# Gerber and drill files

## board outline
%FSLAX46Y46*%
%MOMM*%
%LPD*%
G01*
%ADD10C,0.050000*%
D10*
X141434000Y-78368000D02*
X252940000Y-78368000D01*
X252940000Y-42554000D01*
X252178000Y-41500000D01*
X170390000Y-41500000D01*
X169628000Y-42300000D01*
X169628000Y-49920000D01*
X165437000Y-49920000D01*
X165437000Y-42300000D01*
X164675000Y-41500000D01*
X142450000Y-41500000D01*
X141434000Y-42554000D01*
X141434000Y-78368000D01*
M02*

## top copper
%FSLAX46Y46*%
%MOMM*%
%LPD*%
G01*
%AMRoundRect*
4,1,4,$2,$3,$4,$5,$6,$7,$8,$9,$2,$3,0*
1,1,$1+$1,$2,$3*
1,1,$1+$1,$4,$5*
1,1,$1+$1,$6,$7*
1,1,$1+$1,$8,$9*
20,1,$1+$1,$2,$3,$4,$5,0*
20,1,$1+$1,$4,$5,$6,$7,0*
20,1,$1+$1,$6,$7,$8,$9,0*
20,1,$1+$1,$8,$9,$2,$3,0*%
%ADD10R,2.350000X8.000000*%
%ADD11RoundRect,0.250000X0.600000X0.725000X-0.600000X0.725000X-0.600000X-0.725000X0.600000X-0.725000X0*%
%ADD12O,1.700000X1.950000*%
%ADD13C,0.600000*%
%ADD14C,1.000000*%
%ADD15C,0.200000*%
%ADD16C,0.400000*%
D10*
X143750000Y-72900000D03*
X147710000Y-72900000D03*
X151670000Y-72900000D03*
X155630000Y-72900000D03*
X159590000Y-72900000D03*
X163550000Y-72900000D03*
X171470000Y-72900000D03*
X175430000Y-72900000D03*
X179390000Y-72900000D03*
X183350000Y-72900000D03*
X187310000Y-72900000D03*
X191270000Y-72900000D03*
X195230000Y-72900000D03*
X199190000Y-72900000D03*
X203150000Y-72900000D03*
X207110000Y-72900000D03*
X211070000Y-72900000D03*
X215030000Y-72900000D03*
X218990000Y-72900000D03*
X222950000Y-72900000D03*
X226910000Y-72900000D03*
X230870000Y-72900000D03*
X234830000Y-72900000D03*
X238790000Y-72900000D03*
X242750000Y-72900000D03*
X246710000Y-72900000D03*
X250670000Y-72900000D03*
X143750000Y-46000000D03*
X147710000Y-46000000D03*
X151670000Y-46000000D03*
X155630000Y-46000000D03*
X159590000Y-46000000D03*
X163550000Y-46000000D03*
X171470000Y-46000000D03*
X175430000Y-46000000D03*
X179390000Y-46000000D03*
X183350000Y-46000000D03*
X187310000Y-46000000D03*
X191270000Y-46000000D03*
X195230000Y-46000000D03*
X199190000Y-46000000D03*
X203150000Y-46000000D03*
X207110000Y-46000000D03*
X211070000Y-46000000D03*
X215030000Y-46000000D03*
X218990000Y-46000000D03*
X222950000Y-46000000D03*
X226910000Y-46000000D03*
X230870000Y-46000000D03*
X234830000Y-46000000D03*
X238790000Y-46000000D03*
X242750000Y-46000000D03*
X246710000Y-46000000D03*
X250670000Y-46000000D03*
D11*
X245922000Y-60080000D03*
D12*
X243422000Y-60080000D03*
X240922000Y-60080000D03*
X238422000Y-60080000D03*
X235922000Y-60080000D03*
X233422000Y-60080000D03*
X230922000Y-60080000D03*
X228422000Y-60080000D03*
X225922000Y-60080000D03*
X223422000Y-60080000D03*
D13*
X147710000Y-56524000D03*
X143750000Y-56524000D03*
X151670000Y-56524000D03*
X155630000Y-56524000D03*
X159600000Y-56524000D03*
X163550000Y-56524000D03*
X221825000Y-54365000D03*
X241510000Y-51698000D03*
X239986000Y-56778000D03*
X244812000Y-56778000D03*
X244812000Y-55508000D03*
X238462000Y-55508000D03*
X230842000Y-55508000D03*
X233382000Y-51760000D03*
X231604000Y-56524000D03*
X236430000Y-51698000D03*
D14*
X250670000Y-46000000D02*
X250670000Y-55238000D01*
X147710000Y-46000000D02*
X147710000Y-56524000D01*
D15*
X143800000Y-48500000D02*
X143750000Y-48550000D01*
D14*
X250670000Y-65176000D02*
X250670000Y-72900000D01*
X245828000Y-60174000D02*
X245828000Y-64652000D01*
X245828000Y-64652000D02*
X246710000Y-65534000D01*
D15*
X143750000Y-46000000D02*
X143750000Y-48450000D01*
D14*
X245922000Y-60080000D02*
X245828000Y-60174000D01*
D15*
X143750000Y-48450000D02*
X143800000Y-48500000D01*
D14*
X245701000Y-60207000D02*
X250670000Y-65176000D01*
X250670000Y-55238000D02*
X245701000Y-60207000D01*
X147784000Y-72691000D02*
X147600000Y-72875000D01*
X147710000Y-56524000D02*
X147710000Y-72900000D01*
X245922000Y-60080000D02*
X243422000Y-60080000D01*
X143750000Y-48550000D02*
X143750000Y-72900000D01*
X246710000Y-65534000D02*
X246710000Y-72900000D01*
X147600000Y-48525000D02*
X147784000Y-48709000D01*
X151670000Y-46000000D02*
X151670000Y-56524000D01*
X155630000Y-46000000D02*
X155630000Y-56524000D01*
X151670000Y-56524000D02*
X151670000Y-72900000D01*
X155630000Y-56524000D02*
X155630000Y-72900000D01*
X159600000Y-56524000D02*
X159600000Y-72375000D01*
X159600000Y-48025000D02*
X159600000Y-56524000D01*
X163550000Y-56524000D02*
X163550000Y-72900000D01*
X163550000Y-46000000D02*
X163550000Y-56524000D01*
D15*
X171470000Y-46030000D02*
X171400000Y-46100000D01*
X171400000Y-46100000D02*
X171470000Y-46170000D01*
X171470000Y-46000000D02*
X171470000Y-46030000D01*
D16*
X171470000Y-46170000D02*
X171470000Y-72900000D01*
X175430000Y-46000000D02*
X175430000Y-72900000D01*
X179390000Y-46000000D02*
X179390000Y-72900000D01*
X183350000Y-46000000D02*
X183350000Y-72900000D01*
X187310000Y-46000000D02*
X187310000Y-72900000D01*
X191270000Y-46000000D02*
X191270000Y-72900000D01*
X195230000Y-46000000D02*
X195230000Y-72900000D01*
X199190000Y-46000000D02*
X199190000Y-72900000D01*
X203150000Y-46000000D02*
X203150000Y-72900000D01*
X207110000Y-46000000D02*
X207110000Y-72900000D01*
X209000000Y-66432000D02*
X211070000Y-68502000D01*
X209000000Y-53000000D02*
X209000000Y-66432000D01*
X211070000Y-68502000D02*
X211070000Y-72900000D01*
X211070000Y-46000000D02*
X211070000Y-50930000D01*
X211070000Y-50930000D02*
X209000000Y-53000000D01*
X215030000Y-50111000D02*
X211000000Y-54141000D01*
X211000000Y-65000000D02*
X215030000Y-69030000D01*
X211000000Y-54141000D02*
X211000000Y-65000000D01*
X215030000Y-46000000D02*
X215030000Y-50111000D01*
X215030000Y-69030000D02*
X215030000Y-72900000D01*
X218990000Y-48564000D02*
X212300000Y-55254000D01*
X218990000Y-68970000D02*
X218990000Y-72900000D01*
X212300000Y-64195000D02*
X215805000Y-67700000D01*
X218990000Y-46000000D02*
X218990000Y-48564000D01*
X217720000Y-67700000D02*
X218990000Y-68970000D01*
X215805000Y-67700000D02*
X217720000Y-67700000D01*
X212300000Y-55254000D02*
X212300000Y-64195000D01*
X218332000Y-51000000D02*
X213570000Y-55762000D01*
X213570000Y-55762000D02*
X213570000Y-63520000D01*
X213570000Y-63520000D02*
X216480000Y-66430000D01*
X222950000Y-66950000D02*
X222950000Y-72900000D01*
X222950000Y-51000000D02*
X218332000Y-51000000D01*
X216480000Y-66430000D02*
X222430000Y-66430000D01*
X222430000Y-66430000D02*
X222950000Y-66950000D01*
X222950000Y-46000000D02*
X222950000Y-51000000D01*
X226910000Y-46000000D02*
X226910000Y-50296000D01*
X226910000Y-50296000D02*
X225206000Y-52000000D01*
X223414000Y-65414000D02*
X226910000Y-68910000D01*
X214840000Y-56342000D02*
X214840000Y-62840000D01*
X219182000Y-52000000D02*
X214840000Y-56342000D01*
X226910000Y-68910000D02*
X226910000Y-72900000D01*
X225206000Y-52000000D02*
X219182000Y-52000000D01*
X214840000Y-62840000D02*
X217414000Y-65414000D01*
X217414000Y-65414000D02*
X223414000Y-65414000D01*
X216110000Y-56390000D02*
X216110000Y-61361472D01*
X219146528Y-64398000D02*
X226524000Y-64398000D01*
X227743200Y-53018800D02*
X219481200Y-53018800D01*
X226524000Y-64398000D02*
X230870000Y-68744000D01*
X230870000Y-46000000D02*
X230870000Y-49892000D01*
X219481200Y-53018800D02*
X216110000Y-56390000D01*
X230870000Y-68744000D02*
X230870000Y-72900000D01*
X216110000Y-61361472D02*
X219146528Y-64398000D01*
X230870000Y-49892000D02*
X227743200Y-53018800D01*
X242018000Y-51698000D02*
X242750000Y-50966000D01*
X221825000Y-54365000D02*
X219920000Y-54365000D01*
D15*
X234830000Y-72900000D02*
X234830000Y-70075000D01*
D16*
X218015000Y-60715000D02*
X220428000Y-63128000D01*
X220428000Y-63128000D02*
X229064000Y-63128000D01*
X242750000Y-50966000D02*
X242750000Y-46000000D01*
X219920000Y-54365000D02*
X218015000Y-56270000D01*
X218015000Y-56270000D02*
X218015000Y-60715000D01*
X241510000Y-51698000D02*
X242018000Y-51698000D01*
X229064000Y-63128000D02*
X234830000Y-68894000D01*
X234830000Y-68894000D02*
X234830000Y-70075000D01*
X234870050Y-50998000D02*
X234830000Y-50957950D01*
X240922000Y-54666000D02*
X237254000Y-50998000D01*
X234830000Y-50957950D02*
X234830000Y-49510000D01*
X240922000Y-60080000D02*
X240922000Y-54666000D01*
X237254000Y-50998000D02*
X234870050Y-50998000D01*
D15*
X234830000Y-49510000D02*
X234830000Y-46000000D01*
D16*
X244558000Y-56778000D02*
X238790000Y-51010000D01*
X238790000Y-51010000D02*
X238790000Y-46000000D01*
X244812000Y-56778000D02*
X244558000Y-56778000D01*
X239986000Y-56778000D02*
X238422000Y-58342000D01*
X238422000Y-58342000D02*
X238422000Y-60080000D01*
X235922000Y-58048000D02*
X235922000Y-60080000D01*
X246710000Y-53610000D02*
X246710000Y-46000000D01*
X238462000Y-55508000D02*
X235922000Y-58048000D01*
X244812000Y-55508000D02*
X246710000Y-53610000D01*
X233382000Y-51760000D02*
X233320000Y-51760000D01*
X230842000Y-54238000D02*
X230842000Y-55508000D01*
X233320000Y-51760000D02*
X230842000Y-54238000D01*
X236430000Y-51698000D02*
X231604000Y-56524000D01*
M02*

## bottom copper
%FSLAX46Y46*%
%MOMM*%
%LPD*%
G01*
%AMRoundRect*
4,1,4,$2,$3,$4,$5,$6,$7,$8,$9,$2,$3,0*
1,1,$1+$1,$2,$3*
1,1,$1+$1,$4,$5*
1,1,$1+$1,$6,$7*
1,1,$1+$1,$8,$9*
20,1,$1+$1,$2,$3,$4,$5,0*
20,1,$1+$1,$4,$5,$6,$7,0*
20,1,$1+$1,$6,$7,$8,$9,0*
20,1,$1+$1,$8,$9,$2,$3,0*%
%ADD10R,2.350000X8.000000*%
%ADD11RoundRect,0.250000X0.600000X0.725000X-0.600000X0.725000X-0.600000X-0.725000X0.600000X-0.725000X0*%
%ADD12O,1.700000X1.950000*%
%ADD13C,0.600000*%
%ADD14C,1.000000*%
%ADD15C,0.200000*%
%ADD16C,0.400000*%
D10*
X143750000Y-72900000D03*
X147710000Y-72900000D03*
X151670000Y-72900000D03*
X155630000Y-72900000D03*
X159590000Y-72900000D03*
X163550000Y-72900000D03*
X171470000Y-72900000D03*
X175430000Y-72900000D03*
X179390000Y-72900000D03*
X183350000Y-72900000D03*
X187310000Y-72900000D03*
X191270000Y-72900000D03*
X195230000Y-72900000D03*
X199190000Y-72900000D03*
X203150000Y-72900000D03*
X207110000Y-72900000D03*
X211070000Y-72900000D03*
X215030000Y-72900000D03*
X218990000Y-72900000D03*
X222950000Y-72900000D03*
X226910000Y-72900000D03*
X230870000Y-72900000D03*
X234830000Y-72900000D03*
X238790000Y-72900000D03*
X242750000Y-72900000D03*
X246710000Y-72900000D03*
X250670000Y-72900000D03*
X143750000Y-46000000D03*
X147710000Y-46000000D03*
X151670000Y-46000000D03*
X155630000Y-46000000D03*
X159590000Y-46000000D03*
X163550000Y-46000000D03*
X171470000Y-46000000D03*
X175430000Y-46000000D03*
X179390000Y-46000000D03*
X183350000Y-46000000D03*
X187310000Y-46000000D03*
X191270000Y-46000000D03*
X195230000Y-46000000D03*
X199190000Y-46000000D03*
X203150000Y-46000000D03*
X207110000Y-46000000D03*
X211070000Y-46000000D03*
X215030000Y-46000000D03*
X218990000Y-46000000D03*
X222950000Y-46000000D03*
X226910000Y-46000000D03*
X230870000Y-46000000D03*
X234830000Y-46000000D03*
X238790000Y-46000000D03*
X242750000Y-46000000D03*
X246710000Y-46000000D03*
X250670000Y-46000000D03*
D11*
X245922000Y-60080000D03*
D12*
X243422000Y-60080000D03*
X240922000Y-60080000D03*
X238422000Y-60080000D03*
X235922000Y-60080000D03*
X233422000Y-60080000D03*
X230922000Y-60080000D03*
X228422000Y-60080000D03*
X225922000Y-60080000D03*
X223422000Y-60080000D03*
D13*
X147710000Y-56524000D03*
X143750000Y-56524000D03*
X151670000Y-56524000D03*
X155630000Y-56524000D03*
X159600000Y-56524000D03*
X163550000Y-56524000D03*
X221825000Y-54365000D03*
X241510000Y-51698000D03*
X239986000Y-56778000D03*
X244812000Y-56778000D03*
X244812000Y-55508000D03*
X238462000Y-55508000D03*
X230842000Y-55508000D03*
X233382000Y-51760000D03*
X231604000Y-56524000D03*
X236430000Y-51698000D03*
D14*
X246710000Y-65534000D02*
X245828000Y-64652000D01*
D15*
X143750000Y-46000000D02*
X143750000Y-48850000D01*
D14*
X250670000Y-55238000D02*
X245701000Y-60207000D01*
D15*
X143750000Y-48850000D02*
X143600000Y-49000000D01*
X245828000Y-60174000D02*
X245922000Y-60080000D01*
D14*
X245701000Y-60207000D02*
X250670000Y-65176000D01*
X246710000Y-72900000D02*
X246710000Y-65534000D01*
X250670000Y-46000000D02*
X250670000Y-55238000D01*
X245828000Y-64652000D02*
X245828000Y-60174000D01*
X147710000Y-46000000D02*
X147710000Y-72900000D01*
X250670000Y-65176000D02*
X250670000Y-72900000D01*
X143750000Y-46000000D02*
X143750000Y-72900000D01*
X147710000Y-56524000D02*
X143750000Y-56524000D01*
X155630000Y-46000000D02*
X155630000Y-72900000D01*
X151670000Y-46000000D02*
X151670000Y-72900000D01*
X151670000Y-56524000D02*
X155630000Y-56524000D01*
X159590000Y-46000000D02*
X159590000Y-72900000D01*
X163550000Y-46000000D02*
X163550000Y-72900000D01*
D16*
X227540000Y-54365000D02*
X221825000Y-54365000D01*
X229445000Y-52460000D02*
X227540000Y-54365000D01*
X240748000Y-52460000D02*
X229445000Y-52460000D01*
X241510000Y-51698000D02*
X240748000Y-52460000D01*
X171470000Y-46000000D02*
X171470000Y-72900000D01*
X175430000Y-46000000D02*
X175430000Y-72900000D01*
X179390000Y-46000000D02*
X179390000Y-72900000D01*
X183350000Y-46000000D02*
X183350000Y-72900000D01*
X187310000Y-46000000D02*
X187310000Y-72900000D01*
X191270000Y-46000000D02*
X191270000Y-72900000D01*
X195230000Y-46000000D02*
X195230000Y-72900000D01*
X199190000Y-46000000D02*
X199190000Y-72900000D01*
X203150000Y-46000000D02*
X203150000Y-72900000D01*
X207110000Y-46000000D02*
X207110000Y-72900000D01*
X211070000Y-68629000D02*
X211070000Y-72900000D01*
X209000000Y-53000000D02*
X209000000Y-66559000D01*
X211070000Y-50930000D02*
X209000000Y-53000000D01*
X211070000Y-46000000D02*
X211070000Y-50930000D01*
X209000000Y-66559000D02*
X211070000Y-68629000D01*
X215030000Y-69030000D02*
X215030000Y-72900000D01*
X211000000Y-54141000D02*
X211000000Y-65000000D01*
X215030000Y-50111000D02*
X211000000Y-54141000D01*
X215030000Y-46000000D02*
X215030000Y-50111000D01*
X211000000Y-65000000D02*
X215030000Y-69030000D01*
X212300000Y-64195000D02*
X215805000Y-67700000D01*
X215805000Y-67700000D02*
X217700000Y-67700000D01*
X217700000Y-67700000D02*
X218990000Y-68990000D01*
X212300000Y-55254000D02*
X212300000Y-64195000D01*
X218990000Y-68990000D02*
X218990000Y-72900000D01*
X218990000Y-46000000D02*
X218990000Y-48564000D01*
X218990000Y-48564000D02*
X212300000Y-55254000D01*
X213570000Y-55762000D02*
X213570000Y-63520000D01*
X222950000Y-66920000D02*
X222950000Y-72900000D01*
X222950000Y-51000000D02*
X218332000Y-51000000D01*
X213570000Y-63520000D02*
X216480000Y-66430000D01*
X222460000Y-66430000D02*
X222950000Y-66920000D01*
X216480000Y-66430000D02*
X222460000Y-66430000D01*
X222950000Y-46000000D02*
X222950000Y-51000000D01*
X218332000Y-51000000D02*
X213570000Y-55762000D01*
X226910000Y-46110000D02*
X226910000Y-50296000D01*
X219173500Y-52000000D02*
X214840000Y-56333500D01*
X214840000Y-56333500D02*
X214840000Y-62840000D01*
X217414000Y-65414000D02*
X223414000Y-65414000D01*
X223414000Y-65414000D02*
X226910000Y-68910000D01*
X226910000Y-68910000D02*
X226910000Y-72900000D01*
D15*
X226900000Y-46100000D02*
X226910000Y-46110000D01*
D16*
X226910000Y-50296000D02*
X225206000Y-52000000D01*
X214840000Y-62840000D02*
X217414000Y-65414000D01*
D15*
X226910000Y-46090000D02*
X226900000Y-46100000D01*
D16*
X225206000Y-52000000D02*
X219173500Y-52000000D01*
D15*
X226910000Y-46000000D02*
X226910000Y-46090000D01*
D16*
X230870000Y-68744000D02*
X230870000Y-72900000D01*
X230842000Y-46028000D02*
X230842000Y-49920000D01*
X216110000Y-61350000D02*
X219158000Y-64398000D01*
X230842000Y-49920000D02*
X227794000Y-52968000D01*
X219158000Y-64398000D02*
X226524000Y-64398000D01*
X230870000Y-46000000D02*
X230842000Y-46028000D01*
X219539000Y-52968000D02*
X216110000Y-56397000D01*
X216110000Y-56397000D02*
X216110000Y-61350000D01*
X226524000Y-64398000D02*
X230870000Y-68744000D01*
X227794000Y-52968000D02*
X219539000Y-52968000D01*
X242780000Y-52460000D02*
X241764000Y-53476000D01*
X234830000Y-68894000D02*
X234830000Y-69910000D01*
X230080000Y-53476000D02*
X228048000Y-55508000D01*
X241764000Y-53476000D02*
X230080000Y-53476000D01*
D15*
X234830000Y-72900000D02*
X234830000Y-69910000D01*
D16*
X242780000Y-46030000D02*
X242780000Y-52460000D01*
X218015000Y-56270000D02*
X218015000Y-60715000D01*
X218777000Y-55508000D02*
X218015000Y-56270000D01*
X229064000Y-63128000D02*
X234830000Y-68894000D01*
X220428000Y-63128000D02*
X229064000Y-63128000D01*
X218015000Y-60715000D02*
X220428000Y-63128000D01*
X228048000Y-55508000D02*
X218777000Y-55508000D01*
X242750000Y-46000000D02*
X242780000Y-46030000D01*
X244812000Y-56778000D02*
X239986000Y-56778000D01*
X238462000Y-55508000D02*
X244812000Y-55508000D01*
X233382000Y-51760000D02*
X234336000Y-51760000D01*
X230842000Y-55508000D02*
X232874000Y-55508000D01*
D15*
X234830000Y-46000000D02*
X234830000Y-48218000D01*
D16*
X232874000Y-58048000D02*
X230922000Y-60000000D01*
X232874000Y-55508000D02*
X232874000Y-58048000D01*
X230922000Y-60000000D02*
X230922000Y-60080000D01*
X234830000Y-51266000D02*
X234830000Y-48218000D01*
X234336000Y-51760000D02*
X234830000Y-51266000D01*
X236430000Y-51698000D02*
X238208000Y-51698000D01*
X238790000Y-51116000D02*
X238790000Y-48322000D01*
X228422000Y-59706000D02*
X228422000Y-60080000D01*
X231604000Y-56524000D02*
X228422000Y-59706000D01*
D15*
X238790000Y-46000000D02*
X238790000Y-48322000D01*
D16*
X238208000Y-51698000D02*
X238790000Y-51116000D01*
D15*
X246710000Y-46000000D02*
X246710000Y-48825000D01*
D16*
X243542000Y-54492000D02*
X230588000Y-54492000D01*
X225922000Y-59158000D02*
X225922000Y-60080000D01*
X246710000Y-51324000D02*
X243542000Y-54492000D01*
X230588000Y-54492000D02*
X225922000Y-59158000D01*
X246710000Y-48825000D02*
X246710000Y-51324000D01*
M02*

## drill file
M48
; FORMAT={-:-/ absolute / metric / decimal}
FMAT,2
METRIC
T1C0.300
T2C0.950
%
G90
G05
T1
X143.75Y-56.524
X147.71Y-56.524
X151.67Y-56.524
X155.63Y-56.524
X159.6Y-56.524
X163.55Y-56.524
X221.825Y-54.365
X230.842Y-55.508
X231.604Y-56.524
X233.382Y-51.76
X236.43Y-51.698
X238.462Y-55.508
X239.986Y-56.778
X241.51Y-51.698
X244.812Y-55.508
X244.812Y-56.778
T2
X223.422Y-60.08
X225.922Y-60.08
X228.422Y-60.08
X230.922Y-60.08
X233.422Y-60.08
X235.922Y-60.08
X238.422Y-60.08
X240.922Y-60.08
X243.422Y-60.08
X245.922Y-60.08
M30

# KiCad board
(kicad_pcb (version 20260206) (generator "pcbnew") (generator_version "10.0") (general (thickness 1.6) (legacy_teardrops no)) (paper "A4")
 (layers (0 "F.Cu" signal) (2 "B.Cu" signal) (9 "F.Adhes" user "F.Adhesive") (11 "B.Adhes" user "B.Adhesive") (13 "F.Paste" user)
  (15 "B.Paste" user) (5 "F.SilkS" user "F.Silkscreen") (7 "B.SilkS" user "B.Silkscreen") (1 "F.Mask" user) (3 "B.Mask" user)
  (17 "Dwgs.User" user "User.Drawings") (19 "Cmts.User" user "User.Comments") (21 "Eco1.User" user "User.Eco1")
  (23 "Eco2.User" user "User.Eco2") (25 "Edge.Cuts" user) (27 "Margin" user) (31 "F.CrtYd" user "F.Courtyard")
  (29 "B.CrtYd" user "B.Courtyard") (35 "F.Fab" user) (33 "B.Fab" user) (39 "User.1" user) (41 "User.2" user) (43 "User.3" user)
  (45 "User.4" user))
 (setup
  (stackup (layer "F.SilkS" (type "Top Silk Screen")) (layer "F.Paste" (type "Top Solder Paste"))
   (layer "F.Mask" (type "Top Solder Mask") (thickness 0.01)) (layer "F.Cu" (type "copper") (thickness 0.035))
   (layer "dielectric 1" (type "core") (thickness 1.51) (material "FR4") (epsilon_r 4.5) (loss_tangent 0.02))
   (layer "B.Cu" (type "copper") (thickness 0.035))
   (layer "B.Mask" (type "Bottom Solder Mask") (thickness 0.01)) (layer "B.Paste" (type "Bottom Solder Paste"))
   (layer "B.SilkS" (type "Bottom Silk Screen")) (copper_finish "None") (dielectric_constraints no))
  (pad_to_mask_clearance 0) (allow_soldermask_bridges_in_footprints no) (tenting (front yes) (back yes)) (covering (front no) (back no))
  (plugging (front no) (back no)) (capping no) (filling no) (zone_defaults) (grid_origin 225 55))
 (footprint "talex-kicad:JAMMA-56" (layer "F.Cu") (at 198.21 91.9)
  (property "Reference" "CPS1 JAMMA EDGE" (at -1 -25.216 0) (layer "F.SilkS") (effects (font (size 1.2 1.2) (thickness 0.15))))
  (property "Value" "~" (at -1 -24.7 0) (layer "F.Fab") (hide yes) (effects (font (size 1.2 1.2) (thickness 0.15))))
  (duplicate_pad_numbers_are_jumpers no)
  (pad "1" smd rect (at -54.46 -19) (size 2.35 8) (layers "F.Cu" "F.Mask" "F.Paste") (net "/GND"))
  (pad "2" smd rect (at -50.5 -19) (size 2.35 8) (layers "F.Cu" "F.Mask" "F.Paste") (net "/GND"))
  (pad "3" smd rect (at -46.54 -19) (size 2.35 8) (layers "F.Cu" "F.Mask" "F.Paste") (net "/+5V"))
  (pad "4" smd rect (at -42.58 -19) (size 2.35 8) (layers "F.Cu" "F.Mask" "F.Paste") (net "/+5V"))
  (pad "5" smd rect (at -38.62 -19) (size 2.35 8) (layers "F.Cu" "F.Mask" "F.Paste") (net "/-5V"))
  (pad "6" smd rect (at -34.66 -19) (size 2.35 8) (layers "F.Cu" "F.Mask" "F.Paste") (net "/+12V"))
  (pad "8" smd rect (at -26.74 -19) (size 2.35 8) (layers "F.Cu" "F.Mask" "F.Paste") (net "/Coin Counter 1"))
  (pad "9" smd rect (at -22.78 -19) (size 2.35 8) (layers "F.Cu" "F.Mask" "F.Paste") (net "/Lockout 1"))
  (pad "10" smd rect (at -18.82 -19) (size 2.35 8) (layers "F.Cu" "F.Mask" "F.Paste") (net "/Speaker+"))
  (pad "11" smd rect (at -14.86 -19) (size 2.35 8) (layers "F.Cu" "F.Mask" "F.Paste") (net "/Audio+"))
  (pad "12" smd rect (at -10.9 -19) (size 2.35 8) (layers "F.Cu" "F.Mask" "F.Paste") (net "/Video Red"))
  (pad "13" smd rect (at -6.94 -19) (size 2.35 8) (layers "F.Cu" "F.Mask" "F.Paste") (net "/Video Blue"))
  (pad "14" smd rect (at -2.98 -19) (size 2.35 8) (layers "F.Cu" "F.Mask" "F.Paste") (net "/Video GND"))
  (pad "15" smd rect (at 0.98 -19) (size 2.35 8) (layers "F.Cu" "F.Mask" "F.Paste") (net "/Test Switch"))
  (pad "16" smd rect (at 4.94 -19) (size 2.35 8) (layers "F.Cu" "F.Mask" "F.Paste") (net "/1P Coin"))
  (pad "17" smd rect (at 8.9 -19) (size 2.35 8) (layers "F.Cu" "F.Mask" "F.Paste") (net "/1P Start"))
  (pad "18" smd rect (at 12.86 -19) (size 2.35 8) (layers "F.Cu" "F.Mask" "F.Paste") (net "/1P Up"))
  (pad "19" smd rect (at 16.82 -19) (size 2.35 8) (layers "F.Cu" "F.Mask" "F.Paste") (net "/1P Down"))
  (pad "20" smd rect (at 20.78 -19) (size 2.35 8) (layers "F.Cu" "F.Mask" "F.Paste") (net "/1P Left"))
  (pad "21" smd rect (at 24.74 -19) (size 2.35 8) (layers "F.Cu" "F.Mask" "F.Paste") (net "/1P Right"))
  (pad "22" smd rect (at 28.7 -19) (size 2.35 8) (layers "F.Cu" "F.Mask" "F.Paste") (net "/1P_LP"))
  (pad "23" smd rect (at 32.66 -19) (size 2.35 8) (layers "F.Cu" "F.Mask" "F.Paste") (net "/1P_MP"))
  (pad "24" smd rect (at 36.62 -19) (size 2.35 8) (layers "F.Cu" "F.Mask" "F.Paste") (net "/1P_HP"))
  (pad "25" smd rect (at 40.58 -19) (size 2.35 8) (layers "F.Cu" "F.Mask" "F.Paste") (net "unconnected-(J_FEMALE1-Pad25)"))
  (pad "26" smd rect (at 44.54 -19) (size 2.35 8) (layers "F.Cu" "F.Mask" "F.Paste") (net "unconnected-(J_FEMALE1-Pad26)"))
  (pad "27" smd rect (at 48.5 -19) (size 2.35 8) (layers "F.Cu" "F.Mask" "F.Paste") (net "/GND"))
  (pad "28" smd rect (at 52.46 -19) (size 2.35 8) (layers "F.Cu" "F.Mask" "F.Paste") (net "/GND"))
  (pad "A" smd rect (at -54.46 -19) (size 2.35 8) (layers "B.Cu" "B.Mask" "B.Paste") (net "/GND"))
  (pad "B" smd rect (at -50.5 -19) (size 2.35 8) (layers "B.Cu" "B.Mask" "B.Paste") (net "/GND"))
  (pad "C" smd rect (at -46.54 -19) (size 2.35 8) (layers "B.Cu" "B.Mask" "B.Paste") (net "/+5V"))
  (pad "D" smd rect (at -42.58 -19) (size 2.35 8) (layers "B.Cu" "B.Mask" "B.Paste") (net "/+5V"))
  (pad "E" smd rect (at -38.62 -19) (size 2.35 8) (layers "B.Cu" "B.Mask" "B.Paste") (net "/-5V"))
  (pad "F" smd rect (at -34.66 -19) (size 2.35 8) (layers "B.Cu" "B.Mask" "B.Paste") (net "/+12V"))
  (pad "J" smd rect (at -26.74 -19) (size 2.35 8) (layers "B.Cu" "B.Mask" "B.Paste") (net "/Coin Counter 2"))
  (pad "K" smd rect (at -22.78 -19) (size 2.35 8) (layers "B.Cu" "B.Mask" "B.Paste") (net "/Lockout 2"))
  (pad "L" smd rect (at -18.82 -19) (size 2.35 8) (layers "B.Cu" "B.Mask" "B.Paste") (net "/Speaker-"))
  (pad "M" smd rect (at -14.86 -19) (size 2.35 8) (layers "B.Cu" "B.Mask" "B.Paste") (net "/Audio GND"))
  (pad "N" smd rect (at -10.9 -19) (size 2.35 8) (layers "B.Cu" "B.Mask" "B.Paste") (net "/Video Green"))
  (pad "P" smd rect (at -6.94 -19) (size 2.35 8) (layers "B.Cu" "B.Mask" "B.Paste") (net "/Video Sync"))
  (pad "R" smd rect (at -2.98 -19) (size 2.35 8) (layers "B.Cu" "B.Mask" "B.Paste") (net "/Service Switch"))
  (pad "S" smd rect (at 0.98 -19) (size 2.35 8) (layers "B.Cu" "B.Mask" "B.Paste") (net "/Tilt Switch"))
  (pad "T" smd rect (at 4.94 -19) (size 2.35 8) (layers "B.Cu" "B.Mask" "B.Paste") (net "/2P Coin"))
  (pad "U" smd rect (at 8.9 -19) (size 2.35 8) (layers "B.Cu" "B.Mask" "B.Paste") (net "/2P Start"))
  (pad "V" smd rect (at 12.86 -19) (size 2.35 8) (layers "B.Cu" "B.Mask" "B.Paste") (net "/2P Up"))
  (pad "W" smd rect (at 16.82 -19) (size 2.35 8) (layers "B.Cu" "B.Mask" "B.Paste") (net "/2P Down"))
  (pad "X" smd rect (at 20.78 -19) (size 2.35 8) (layers "B.Cu" "B.Mask" "B.Paste") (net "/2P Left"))
  (pad "Y" smd rect (at 24.74 -19) (size 2.35 8) (layers "B.Cu" "B.Mask" "B.Paste") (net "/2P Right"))
  (pad "Z" smd rect (at 28.7 -19) (size 2.35 8) (layers "B.Cu" "B.Mask" "B.Paste") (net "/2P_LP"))
  (pad "a" smd rect (at 32.66 -19) (size 2.35 8) (layers "B.Cu" "B.Mask" "B.Paste") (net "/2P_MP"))
  (pad "b" smd rect (at 36.62 -19) (size 2.35 8) (layers "B.Cu" "B.Mask" "B.Paste") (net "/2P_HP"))
  (pad "c" smd rect (at 40.58 -19) (size 2.35 8) (layers "B.Cu" "B.Mask" "B.Paste") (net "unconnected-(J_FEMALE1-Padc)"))
  (pad "d" smd rect (at 44.54 -19) (size 2.35 8) (layers "B.Cu" "B.Mask" "B.Paste") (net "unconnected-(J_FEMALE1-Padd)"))
  (pad "e" smd rect (at 48.5 -19) (size 2.35 8) (layers "B.Cu" "B.Mask" "B.Paste") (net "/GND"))
  (pad "f" smd rect (at 52.46 -19) (size 2.35 8) (layers "B.Cu" "B.Mask" "B.Paste") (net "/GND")))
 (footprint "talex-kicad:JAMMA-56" (layer "F.Cu") (at 198.21 65)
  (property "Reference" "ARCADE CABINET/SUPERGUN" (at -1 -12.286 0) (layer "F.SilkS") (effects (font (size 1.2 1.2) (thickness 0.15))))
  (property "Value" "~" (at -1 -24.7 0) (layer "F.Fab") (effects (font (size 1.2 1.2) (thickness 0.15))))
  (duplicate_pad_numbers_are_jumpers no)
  (pad "1" smd rect (at -54.46 -19) (size 2.35 8) (layers "F.Cu" "F.Mask" "F.Paste") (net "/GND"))
  (pad "2" smd rect (at -50.5 -19) (size 2.35 8) (layers "F.Cu" "F.Mask" "F.Paste") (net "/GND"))
  (pad "3" smd rect (at -46.54 -19) (size 2.35 8) (layers "F.Cu" "F.Mask" "F.Paste") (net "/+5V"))
  (pad "4" smd rect (at -42.58 -19) (size 2.35 8) (layers "F.Cu" "F.Mask" "F.Paste") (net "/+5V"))
  (pad "5" smd rect (at -38.62 -19) (size 2.35 8) (layers "F.Cu" "F.Mask" "F.Paste") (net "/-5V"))
  (pad "6" smd rect (at -34.66 -19) (size 2.35 8) (layers "F.Cu" "F.Mask" "F.Paste") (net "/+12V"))
  (pad "8" smd rect (at -26.74 -19) (size 2.35 8) (layers "F.Cu" "F.Mask" "F.Paste") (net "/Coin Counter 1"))
  (pad "9" smd rect (at -22.78 -19) (size 2.35 8) (layers "F.Cu" "F.Mask" "F.Paste") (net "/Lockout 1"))
  (pad "10" smd rect (at -18.82 -19) (size 2.35 8) (layers "F.Cu" "F.Mask" "F.Paste") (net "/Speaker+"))
  (pad "11" smd rect (at -14.86 -19) (size 2.35 8) (layers "F.Cu" "F.Mask" "F.Paste") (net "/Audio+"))
  (pad "12" smd rect (at -10.9 -19) (size 2.35 8) (layers "F.Cu" "F.Mask" "F.Paste") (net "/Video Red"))
  (pad "13" smd rect (at -6.94 -19) (size 2.35 8) (layers "F.Cu" "F.Mask" "F.Paste") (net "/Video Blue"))
  (pad "14" smd rect (at -2.98 -19) (size 2.35 8) (layers "F.Cu" "F.Mask" "F.Paste") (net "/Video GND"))
  (pad "15" smd rect (at 0.98 -19) (size 2.35 8) (layers "F.Cu" "F.Mask" "F.Paste") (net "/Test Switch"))
  (pad "16" smd rect (at 4.94 -19) (size 2.35 8) (layers "F.Cu" "F.Mask" "F.Paste") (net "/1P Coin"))
  (pad "17" smd rect (at 8.9 -19) (size 2.35 8) (layers "F.Cu" "F.Mask" "F.Paste") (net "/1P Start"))
  (pad "18" smd rect (at 12.86 -19) (size 2.35 8) (layers "F.Cu" "F.Mask" "F.Paste") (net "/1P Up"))
  (pad "19" smd rect (at 16.82 -19) (size 2.35 8) (layers "F.Cu" "F.Mask" "F.Paste") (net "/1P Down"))
  (pad "20" smd rect (at 20.78 -19) (size 2.35 8) (layers "F.Cu" "F.Mask" "F.Paste") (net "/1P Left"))
  (pad "21" smd rect (at 24.74 -19) (size 2.35 8) (layers "F.Cu" "F.Mask" "F.Paste") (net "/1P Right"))
  (pad "22" smd rect (at 28.7 -19) (size 2.35 8) (layers "F.Cu" "F.Mask" "F.Paste") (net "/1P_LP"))
  (pad "23" smd rect (at 32.66 -19) (size 2.35 8) (layers "F.Cu" "F.Mask" "F.Paste") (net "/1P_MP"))
  (pad "24" smd rect (at 36.62 -19) (size 2.35 8) (layers "F.Cu" "F.Mask" "F.Paste") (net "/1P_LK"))
  (pad "25" smd rect (at 40.58 -19) (size 2.35 8) (layers "F.Cu" "F.Mask" "F.Paste") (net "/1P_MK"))
  (pad "26" smd rect (at 44.54 -19) (size 2.35 8) (layers "F.Cu" "F.Mask" "F.Paste") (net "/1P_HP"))
  (pad "27" smd rect (at 48.5 -19) (size 2.35 8) (layers "F.Cu" "F.Mask" "F.Paste") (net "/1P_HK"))
  (pad "28" smd rect (at 52.46 -19) (size 2.35 8) (layers "F.Cu" "F.Mask" "F.Paste") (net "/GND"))
  (pad "A" smd rect (at -54.46 -19) (size 2.35 8) (layers "B.Cu" "B.Mask" "B.Paste") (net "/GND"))
  (pad "B" smd rect (at -50.5 -19) (size 2.35 8) (layers "B.Cu" "B.Mask" "B.Paste") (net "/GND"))
  (pad "C" smd rect (at -46.54 -19) (size 2.35 8) (layers "B.Cu" "B.Mask" "B.Paste") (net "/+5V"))
  (pad "D" smd rect (at -42.58 -19) (size 2.35 8) (layers "B.Cu" "B.Mask" "B.Paste") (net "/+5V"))
  (pad "E" smd rect (at -38.62 -19) (size 2.35 8) (layers "B.Cu" "B.Mask" "B.Paste") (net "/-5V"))
  (pad "F" smd rect (at -34.66 -19) (size 2.35 8) (layers "B.Cu" "B.Mask" "B.Paste") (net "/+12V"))
  (pad "J" smd rect (at -26.74 -19) (size 2.35 8) (layers "B.Cu" "B.Mask" "B.Paste") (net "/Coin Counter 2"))
  (pad "K" smd rect (at -22.78 -19) (size 2.35 8) (layers "B.Cu" "B.Mask" "B.Paste") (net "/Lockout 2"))
  (pad "L" smd rect (at -18.82 -19) (size 2.35 8) (layers "B.Cu" "B.Mask" "B.Paste") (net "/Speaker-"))
  (pad "M" smd rect (at -14.86 -19) (size 2.35 8) (layers "B.Cu" "B.Mask" "B.Paste") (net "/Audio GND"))
  (pad "N" smd rect (at -10.9 -19) (size 2.35 8) (layers "B.Cu" "B.Mask" "B.Paste") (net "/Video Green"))
  (pad "P" smd rect (at -6.94 -19) (size 2.35 8) (layers "B.Cu" "B.Mask" "B.Paste") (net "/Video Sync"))
  (pad "R" smd rect (at -2.98 -19) (size 2.35 8) (layers "B.Cu" "B.Mask" "B.Paste") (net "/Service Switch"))
  (pad "S" smd rect (at 0.98 -19) (size 2.35 8) (layers "B.Cu" "B.Mask" "B.Paste") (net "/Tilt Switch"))
  (pad "T" smd rect (at 4.94 -19) (size 2.35 8) (layers "B.Cu" "B.Mask" "B.Paste") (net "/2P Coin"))
  (pad "U" smd rect (at 8.9 -19) (size 2.35 8) (layers "B.Cu" "B.Mask" "B.Paste") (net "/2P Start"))
  (pad "V" smd rect (at 12.86 -19) (size 2.35 8) (layers "B.Cu" "B.Mask" "B.Paste") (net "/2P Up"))
  (pad "W" smd rect (at 16.82 -19) (size 2.35 8) (layers "B.Cu" "B.Mask" "B.Paste") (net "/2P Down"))
  (pad "X" smd rect (at 20.78 -19) (size 2.35 8) (layers "B.Cu" "B.Mask" "B.Paste") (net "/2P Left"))
  (pad "Y" smd rect (at 24.74 -19) (size 2.35 8) (layers "B.Cu" "B.Mask" "B.Paste") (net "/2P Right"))
  (pad "Z" smd rect (at 28.7 -19) (size 2.35 8) (layers "B.Cu" "B.Mask" "B.Paste") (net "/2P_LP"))
  (pad "a" smd rect (at 32.66 -19) (size 2.35 8) (layers "B.Cu" "B.Mask" "B.Paste") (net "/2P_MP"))
  (pad "b" smd rect (at 36.62 -19) (size 2.35 8) (layers "B.Cu" "B.Mask" "B.Paste") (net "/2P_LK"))
  (pad "c" smd rect (at 40.58 -19) (size 2.35 8) (layers "B.Cu" "B.Mask" "B.Paste") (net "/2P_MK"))
  (pad "d" smd rect (at 44.54 -19) (size 2.35 8) (layers "B.Cu" "B.Mask" "B.Paste") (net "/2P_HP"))
  (pad "e" smd rect (at 48.5 -19) (size 2.35 8) (layers "B.Cu" "B.Mask" "B.Paste") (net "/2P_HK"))
  (pad "f" smd rect (at 52.46 -19) (size 2.35 8) (layers "B.Cu" "B.Mask" "B.Paste") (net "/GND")))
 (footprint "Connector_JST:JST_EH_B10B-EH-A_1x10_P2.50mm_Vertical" (layer "F.Cu") (at 245.922 60.08 180)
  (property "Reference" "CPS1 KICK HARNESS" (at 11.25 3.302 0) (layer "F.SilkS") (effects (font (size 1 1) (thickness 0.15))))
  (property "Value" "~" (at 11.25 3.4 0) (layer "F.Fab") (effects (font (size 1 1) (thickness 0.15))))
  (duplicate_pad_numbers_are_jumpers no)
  (pad "1" thru_hole roundrect (at 0 0 180) (size 1.7 1.95) (drill 0.95) (layers "*.Cu" "*.Mask") (remove_unused_layers no)
   (roundrect_rratio 0.147059) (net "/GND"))
  (pad "2" thru_hole oval (at 2.5 0 180) (size 1.7 1.95) (drill 0.95) (layers "*.Cu" "*.Mask") (remove_unused_layers no) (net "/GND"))
  (pad "3" thru_hole oval (at 5 0 180) (size 1.7 1.95) (drill 0.95) (layers "*.Cu" "*.Mask") (remove_unused_layers no) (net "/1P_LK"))
  (pad "4" thru_hole oval (at 7.5 0 180) (size 1.7 1.95) (drill 0.95) (layers "*.Cu" "*.Mask") (remove_unused_layers no) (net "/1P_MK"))
  (pad "5" thru_hole oval (at 10 0 180) (size 1.7 1.95) (drill 0.95) (layers "*.Cu" "*.Mask") (remove_unused_layers no) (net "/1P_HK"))
  (pad "6" thru_hole oval (at 12.5 0 180) (size 1.7 1.95) (drill 0.95) (layers "*.Cu" "*.Mask") (remove_unused_layers no)
   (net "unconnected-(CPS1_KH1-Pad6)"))
  (pad "7" thru_hole oval (at 15 0 180) (size 1.7 1.95) (drill 0.95) (layers "*.Cu" "*.Mask") (remove_unused_layers no) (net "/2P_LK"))
  (pad "8" thru_hole oval (at 17.5 0 180) (size 1.7 1.95) (drill 0.95) (layers "*.Cu" "*.Mask") (remove_unused_layers no) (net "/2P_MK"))
  (pad "9" thru_hole oval (at 20 0 180) (size 1.7 1.95) (drill 0.95) (layers "*.Cu" "*.Mask") (remove_unused_layers no) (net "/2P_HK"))
  (pad "10" thru_hole oval (at 22.5 0 180) (size 1.7 1.95) (drill 0.95) (layers "*.Cu" "*.Mask") (remove_unused_layers no)
   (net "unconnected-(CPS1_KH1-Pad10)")))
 (gr_poly
  (pts (xy 141.434 78.368) (xy 252.94 78.368) (xy 252.94 42.554) (xy 252.178 41.5) (xy 170.39 41.5) (xy 169.628 42.3) (xy 169.628 49.92)
   (xy 165.437 49.92) (xy 165.437 42.3) (xy 164.675 41.5) (xy 142.45 41.5) (xy 141.434 42.554))
  (stroke (width 0.05) (type solid)) (fill no) (layer "Edge.Cuts"))
 (segment (start 250.67 46) (end 250.67 55.238) (width 1) (layer "F.Cu") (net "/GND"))
 (segment (start 147.71 46) (end 147.71 56.524) (width 1) (layer "F.Cu") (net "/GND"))
 (segment (start 143.8 48.5) (end 143.75 48.55) (width 0.2) (layer "F.Cu") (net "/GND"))
 (segment (start 250.67 65.176) (end 250.67 72.9) (width 1) (layer "F.Cu") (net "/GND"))
 (segment (start 245.828 60.174) (end 245.828 64.652) (width 1) (layer "F.Cu") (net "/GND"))
 (segment (start 245.828 64.652) (end 246.71 65.534) (width 1) (layer "F.Cu") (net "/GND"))
 (segment (start 143.75 46) (end 143.75 48.45) (width 0.2) (layer "F.Cu") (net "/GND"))
 (segment (start 245.922 60.08) (end 245.828 60.174) (width 1) (layer "F.Cu") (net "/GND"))
 (segment (start 143.75 48.45) (end 143.8 48.5) (width 0.2) (layer "F.Cu") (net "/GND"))
 (segment (start 245.701 60.207) (end 250.67 65.176) (width 1) (layer "F.Cu") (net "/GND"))
 (segment (start 250.67 55.238) (end 245.701 60.207) (width 1) (layer "F.Cu") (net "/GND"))
 (segment (start 147.784 72.691) (end 147.6 72.875) (width 1) (layer "F.Cu") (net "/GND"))
 (segment (start 147.71 56.524) (end 147.71 72.9) (width 1) (layer "F.Cu") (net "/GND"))
 (segment (start 245.922 60.08) (end 243.422 60.08) (width 1) (layer "F.Cu") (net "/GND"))
 (segment (start 143.75 48.55) (end 143.75 72.9) (width 1) (layer "F.Cu") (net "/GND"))
 (segment (start 246.71 65.534) (end 246.71 72.9) (width 1) (layer "F.Cu") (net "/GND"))
 (segment (start 147.6 48.525) (end 147.784 48.709) (width 1) (layer "F.Cu") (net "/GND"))
 (via (at 147.71 56.524) (size 0.6) (drill 0.3) (layers "F.Cu" "B.Cu") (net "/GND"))
 (via (at 143.75 56.524) (size 0.6) (drill 0.3) (layers "F.Cu" "B.Cu") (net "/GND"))
 (segment (start 246.71 65.534) (end 245.828 64.652) (width 1) (layer "B.Cu") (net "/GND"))
 (segment (start 143.75 46) (end 143.75 48.85) (width 0.2) (layer "B.Cu") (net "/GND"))
 (segment (start 250.67 55.238) (end 245.701 60.207) (width 1) (layer "B.Cu") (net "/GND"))
 (segment (start 143.75 48.85) (end 143.6 49) (width 0.2) (layer "B.Cu") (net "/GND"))
 (segment (start 245.828 60.174) (end 245.922 60.08) (width 0.2) (layer "B.Cu") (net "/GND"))
 (segment (start 245.701 60.207) (end 250.67 65.176) (width 1) (layer "B.Cu") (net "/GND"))
 (segment (start 246.71 72.9) (end 246.71 65.534) (width 1) (layer "B.Cu") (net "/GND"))
 (segment (start 250.67 46) (end 250.67 55.238) (width 1) (layer "B.Cu") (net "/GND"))
 (segment (start 245.828 64.652) (end 245.828 60.174) (width 1) (layer "B.Cu") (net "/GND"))
 (segment (start 147.71 46) (end 147.71 72.9) (width 1) (layer "B.Cu") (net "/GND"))
 (segment (start 250.67 65.176) (end 250.67 72.9) (width 1) (layer "B.Cu") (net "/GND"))
 (segment (start 143.75 46) (end 143.75 72.9) (width 1) (layer "B.Cu") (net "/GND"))
 (segment (start 147.71 56.524) (end 143.75 56.524) (width 1) (layer "B.Cu") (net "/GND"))
 (segment (start 151.67 46) (end 151.67 56.524) (width 1) (layer "F.Cu") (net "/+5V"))
 (segment (start 155.63 46) (end 155.63 56.524) (width 1) (layer "F.Cu") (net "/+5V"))
 (segment (start 151.67 56.524) (end 151.67 72.9) (width 1) (layer "F.Cu") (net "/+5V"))
 (segment (start 155.63 56.524) (end 155.63 72.9) (width 1) (layer "F.Cu") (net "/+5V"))
 (via (at 151.67 56.524) (size 0.6) (drill 0.3) (layers "F.Cu" "B.Cu") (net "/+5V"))
 (via (at 155.63 56.524) (size 0.6) (drill 0.3) (layers "F.Cu" "B.Cu") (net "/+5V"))
 (segment (start 155.63 46) (end 155.63 72.9) (width 1) (layer "B.Cu") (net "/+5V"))
 (segment (start 151.67 46) (end 151.67 72.9) (width 1) (layer "B.Cu") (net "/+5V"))
 (segment (start 151.67 56.524) (end 155.63 56.524) (width 1) (layer "B.Cu") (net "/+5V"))
 (segment (start 159.6 56.524) (end 159.6 72.375) (width 1) (layer "F.Cu") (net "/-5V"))
 (segment (start 159.6 48.025) (end 159.6 56.524) (width 1) (layer "F.Cu") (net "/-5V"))
 (via (at 159.6 56.524) (size 0.6) (drill 0.3) (layers "F.Cu" "B.Cu") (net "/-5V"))
 (segment (start 159.59 46) (end 159.59 72.9) (width 1) (layer "B.Cu") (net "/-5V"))
 (segment (start 163.55 56.524) (end 163.55 72.9) (width 1) (layer "F.Cu") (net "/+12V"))
 (segment (start 163.55 46) (end 163.55 56.524) (width 1) (layer "F.Cu") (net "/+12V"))
 (via (at 163.55 56.524) (size 0.6) (drill 0.3) (layers "F.Cu" "B.Cu") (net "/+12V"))
 (segment (start 163.55 46) (end 163.55 72.9) (width 1) (layer "B.Cu") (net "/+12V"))
 (segment (start 171.47 46.03) (end 171.4 46.1) (width 0.2) (layer "F.Cu") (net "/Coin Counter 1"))
 (segment (start 171.4 46.1) (end 171.47 46.17) (width 0.2) (layer "F.Cu") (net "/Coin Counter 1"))
 (segment (start 171.47 46) (end 171.47 46.03) (width 0.2) (layer "F.Cu") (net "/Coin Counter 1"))
 (segment (start 171.47 46.17) (end 171.47 72.9) (width 0.4) (layer "F.Cu") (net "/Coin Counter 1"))
 (segment (start 175.43 46) (end 175.43 72.9) (width 0.4) (layer "F.Cu") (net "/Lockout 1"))
 (segment (start 179.39 46) (end 179.39 72.9) (width 0.4) (layer "F.Cu") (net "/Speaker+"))
 (segment (start 183.35 46) (end 183.35 72.9) (width 0.4) (layer "F.Cu") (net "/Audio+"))
 (segment (start 187.31 46) (end 187.31 72.9) (width 0.4) (layer "F.Cu") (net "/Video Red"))
 (segment (start 191.27 46) (end 191.27 72.9) (width 0.4) (layer "F.Cu") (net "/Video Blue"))
 (segment (start 195.23 46) (end 195.23 72.9) (width 0.4) (layer "F.Cu") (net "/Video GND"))
 (segment (start 199.19 46) (end 199.19 72.9) (width 0.4) (layer "F.Cu") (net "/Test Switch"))
 (segment (start 203.15 46) (end 203.15 72.9) (width 0.4) (layer "F.Cu") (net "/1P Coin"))
 (segment (start 207.11 46) (end 207.11 72.9) (width 0.4) (layer "F.Cu") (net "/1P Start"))
 (segment (start 209 66.432) (end 211.07 68.502) (width 0.4) (layer "F.Cu") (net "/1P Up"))
 (segment (start 209 53) (end 209 66.432) (width 0.4) (layer "F.Cu") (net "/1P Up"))
 (segment (start 211.07 68.502) (end 211.07 72.9) (width 0.4) (layer "F.Cu") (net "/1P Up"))
 (segment (start 211.07 46) (end 211.07 50.93) (width 0.4) (layer "F.Cu") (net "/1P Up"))
 (segment (start 211.07 50.93) (end 209 53) (width 0.4) (layer "F.Cu") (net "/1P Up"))
 (segment (start 215.03 50.111) (end 211 54.141) (width 0.4) (layer "F.Cu") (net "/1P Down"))
 (segment (start 211 65) (end 215.03 69.03) (width 0.4) (layer "F.Cu") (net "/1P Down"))
 (segment (start 211 54.141) (end 211 65) (width 0.4) (layer "F.Cu") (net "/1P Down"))
 (segment (start 215.03 46) (end 215.03 50.111) (width 0.4) (layer "F.Cu") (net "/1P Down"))
 (segment (start 215.03 69.03) (end 215.03 72.9) (width 0.4) (layer "F.Cu") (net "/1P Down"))
 (segment (start 218.99 48.564) (end 212.3 55.254) (width 0.4) (layer "F.Cu") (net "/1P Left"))
 (segment (start 218.99 68.97) (end 218.99 72.9) (width 0.4) (layer "F.Cu") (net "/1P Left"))
 (segment (start 212.3 64.195) (end 215.805 67.7) (width 0.4) (layer "F.Cu") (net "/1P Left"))
 (segment (start 218.99 46) (end 218.99 48.564) (width 0.4) (layer "F.Cu") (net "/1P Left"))
 (segment (start 217.72 67.7) (end 218.99 68.97) (width 0.4) (layer "F.Cu") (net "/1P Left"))
 (segment (start 215.805 67.7) (end 217.72 67.7) (width 0.4) (layer "F.Cu") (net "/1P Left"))
 (segment (start 212.3 55.254) (end 212.3 64.195) (width 0.4) (layer "F.Cu") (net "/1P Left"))
 (segment (start 218.332 51) (end 213.57 55.762) (width 0.4) (layer "F.Cu") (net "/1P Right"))
 (segment (start 213.57 55.762) (end 213.57 63.52) (width 0.4) (layer "F.Cu") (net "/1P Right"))
 (segment (start 213.57 63.52) (end 216.48 66.43) (width 0.4) (layer "F.Cu") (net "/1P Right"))
 (segment (start 222.95 66.95) (end 222.95 72.9) (width 0.4) (layer "F.Cu") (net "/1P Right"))
 (segment (start 222.95 51) (end 218.332 51) (width 0.4) (layer "F.Cu") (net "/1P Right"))
 (segment (start 216.48 66.43) (end 222.43 66.43) (width 0.4) (layer "F.Cu") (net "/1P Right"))
 (segment (start 222.43 66.43) (end 222.95 66.95) (width 0.4) (layer "F.Cu") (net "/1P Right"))
 (segment (start 222.95 46) (end 222.95 51) (width 0.4) (layer "F.Cu") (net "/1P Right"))
 (segment (start 226.91 46) (end 226.91 50.296) (width 0.4) (layer "F.Cu") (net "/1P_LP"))
 (segment (start 226.91 50.296) (end 225.206 52) (width 0.4) (layer "F.Cu") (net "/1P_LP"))
 (segment (start 223.414 65.414) (end 226.91 68.91) (width 0.4) (layer "F.Cu") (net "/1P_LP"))
 (segment (start 214.84 56.342) (end 214.84 62.84) (width 0.4) (layer "F.Cu") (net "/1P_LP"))
 (segment (start 219.182 52) (end 214.84 56.342) (width 0.4) (layer "F.Cu") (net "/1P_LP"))
 (segment (start 226.91 68.91) (end 226.91 72.9) (width 0.4) (layer "F.Cu") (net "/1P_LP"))
 (segment (start 225.206 52) (end 219.182 52) (width 0.4) (layer "F.Cu") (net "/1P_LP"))
 (segment (start 214.84 62.84) (end 217.414 65.414) (width 0.4) (layer "F.Cu") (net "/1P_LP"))
 (segment (start 217.414 65.414) (end 223.414 65.414) (width 0.4) (layer "F.Cu") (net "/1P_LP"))
 (segment (start 216.11 56.39) (end 216.11 61.361472) (width 0.4) (layer "F.Cu") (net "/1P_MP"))
 (segment (start 219.146528 64.398) (end 226.524 64.398) (width 0.4) (layer "F.Cu") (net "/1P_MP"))
 (segment (start 227.7432 53.0188) (end 219.4812 53.0188) (width 0.4) (layer "F.Cu") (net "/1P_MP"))
 (segment (start 226.524 64.398) (end 230.87 68.744) (width 0.4) (layer "F.Cu") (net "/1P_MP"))
 (segment (start 230.87 46) (end 230.87 49.892) (width 0.4) (layer "F.Cu") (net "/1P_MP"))
 (segment (start 219.4812 53.0188) (end 216.11 56.39) (width 0.4) (layer "F.Cu") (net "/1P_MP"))
 (segment (start 230.87 68.744) (end 230.87 72.9) (width 0.4) (layer "F.Cu") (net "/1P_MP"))
 (segment (start 216.11 61.361472) (end 219.146528 64.398) (width 0.4) (layer "F.Cu") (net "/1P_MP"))
 (segment (start 230.87 49.892) (end 227.7432 53.0188) (width 0.4) (layer "F.Cu") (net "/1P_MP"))
 (segment (start 242.018 51.698) (end 242.75 50.966) (width 0.4) (layer "F.Cu") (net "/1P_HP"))
 (segment (start 221.825 54.365) (end 219.92 54.365) (width 0.4) (layer "F.Cu") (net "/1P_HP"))
 (segment (start 234.83 72.9) (end 234.83 70.075) (width 0.2) (layer "F.Cu") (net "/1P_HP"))
 (segment (start 218.015 60.715) (end 220.428 63.128) (width 0.4) (layer "F.Cu") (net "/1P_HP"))
 (segment (start 220.428 63.128) (end 229.064 63.128) (width 0.4) (layer "F.Cu") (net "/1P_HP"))
 (segment (start 242.75 50.966) (end 242.75 46) (width 0.4) (layer "F.Cu") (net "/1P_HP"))
 (segment (start 219.92 54.365) (end 218.015 56.27) (width 0.4) (layer "F.Cu") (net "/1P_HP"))
 (segment (start 218.015 56.27) (end 218.015 60.715) (width 0.4) (layer "F.Cu") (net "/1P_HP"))
 (segment (start 241.51 51.698) (end 242.018 51.698) (width 0.4) (layer "F.Cu") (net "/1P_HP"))
 (segment (start 229.064 63.128) (end 234.83 68.894) (width 0.4) (layer "F.Cu") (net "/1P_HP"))
 (segment (start 234.83 68.894) (end 234.83 70.075) (width 0.4) (layer "F.Cu") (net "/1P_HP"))
 (via (at 221.825 54.365) (size 0.6) (drill 0.3) (layers "F.Cu" "B.Cu") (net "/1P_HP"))
 (via (at 241.51 51.698) (size 0.6) (drill 0.3) (layers "F.Cu" "B.Cu") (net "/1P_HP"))
 (segment (start 227.54 54.365) (end 221.825 54.365) (width 0.4) (layer "B.Cu") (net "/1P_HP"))
 (segment (start 229.445 52.46) (end 227.54 54.365) (width 0.4) (layer "B.Cu") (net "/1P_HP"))
 (segment (start 240.748 52.46) (end 229.445 52.46) (width 0.4) (layer "B.Cu") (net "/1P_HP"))
 (segment (start 241.51 51.698) (end 240.748 52.46) (width 0.4) (layer "B.Cu") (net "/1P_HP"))
 (segment (start 171.47 46) (end 171.47 72.9) (width 0.4) (layer "B.Cu") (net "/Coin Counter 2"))
 (segment (start 175.43 46) (end 175.43 72.9) (width 0.4) (layer "B.Cu") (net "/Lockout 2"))
 (segment (start 179.39 46) (end 179.39 72.9) (width 0.4) (layer "B.Cu") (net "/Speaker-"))
 (segment (start 183.35 46) (end 183.35 72.9) (width 0.4) (layer "B.Cu") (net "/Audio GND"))
 (segment (start 187.31 46) (end 187.31 72.9) (width 0.4) (layer "B.Cu") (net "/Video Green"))
 (segment (start 191.27 46) (end 191.27 72.9) (width 0.4) (layer "B.Cu") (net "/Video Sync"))
 (segment (start 195.23 46) (end 195.23 72.9) (width 0.4) (layer "B.Cu") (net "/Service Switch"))
 (segment (start 199.19 46) (end 199.19 72.9) (width 0.4) (layer "B.Cu") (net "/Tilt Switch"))
 (segment (start 203.15 46) (end 203.15 72.9) (width 0.4) (layer "B.Cu") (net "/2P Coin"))
 (segment (start 207.11 46) (end 207.11 72.9) (width 0.4) (layer "B.Cu") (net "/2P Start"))
 (segment (start 211.07 68.629) (end 211.07 72.9) (width 0.4) (layer "B.Cu") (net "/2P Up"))
 (segment (start 209 53) (end 209 66.559) (width 0.4) (layer "B.Cu") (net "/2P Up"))
 (segment (start 211.07 50.93) (end 209 53) (width 0.4) (layer "B.Cu") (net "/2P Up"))
 (segment (start 211.07 46) (end 211.07 50.93) (width 0.4) (layer "B.Cu") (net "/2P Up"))
 (segment (start 209 66.559) (end 211.07 68.629) (width 0.4) (layer "B.Cu") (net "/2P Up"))
 (segment (start 215.03 69.03) (end 215.03 72.9) (width 0.4) (layer "B.Cu") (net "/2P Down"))
 (segment (start 211 54.141) (end 211 65) (width 0.4) (layer "B.Cu") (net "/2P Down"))
 (segment (start 215.03 50.111) (end 211 54.141) (width 0.4) (layer "B.Cu") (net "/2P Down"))
 (segment (start 215.03 46) (end 215.03 50.111) (width 0.4) (layer "B.Cu") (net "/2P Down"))
 (segment (start 211 65) (end 215.03 69.03) (width 0.4) (layer "B.Cu") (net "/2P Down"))
 (segment (start 212.3 64.195) (end 215.805 67.7) (width 0.4) (layer "B.Cu") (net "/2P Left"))
 (segment (start 215.805 67.7) (end 217.7 67.7) (width 0.4) (layer "B.Cu") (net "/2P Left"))
 (segment (start 217.7 67.7) (end 218.99 68.99) (width 0.4) (layer "B.Cu") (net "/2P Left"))
 (segment (start 212.3 55.254) (end 212.3 64.195) (width 0.4) (layer "B.Cu") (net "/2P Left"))
 (segment (start 218.99 68.99) (end 218.99 72.9) (width 0.4) (layer "B.Cu") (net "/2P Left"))
 (segment (start 218.99 46) (end 218.99 48.564) (width 0.4) (layer "B.Cu") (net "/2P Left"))
 (segment (start 218.99 48.564) (end 212.3 55.254) (width 0.4) (layer "B.Cu") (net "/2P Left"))
 (segment (start 213.57 55.762) (end 213.57 63.52) (width 0.4) (layer "B.Cu") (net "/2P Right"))
 (segment (start 222.95 66.92) (end 222.95 72.9) (width 0.4) (layer "B.Cu") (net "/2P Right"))
 (segment (start 222.95 51) (end 218.332 51) (width 0.4) (layer "B.Cu") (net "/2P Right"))
 (segment (start 213.57 63.52) (end 216.48 66.43) (width 0.4) (layer "B.Cu") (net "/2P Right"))
 (segment (start 222.46 66.43) (end 222.95 66.92) (width 0.4) (layer "B.Cu") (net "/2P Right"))
 (segment (start 216.48 66.43) (end 222.46 66.43) (width 0.4) (layer "B.Cu") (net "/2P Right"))
 (segment (start 222.95 46) (end 222.95 51) (width 0.4) (layer "B.Cu") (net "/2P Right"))
 (segment (start 218.332 51) (end 213.57 55.762) (width 0.4) (layer "B.Cu") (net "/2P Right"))
 (segment (start 226.91 46.11) (end 226.91 50.296) (width 0.4) (layer "B.Cu") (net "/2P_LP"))
 (segment (start 219.1735 52) (end 214.84 56.3335) (width 0.4) (layer "B.Cu") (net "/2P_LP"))
 (segment (start 214.84 56.3335) (end 214.84 62.84) (width 0.4) (layer "B.Cu") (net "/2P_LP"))
 (segment (start 217.414 65.414) (end 223.414 65.414) (width 0.4) (layer "B.Cu") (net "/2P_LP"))
 (segment (start 223.414 65.414) (end 226.91 68.91) (width 0.4) (layer "B.Cu") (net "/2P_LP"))
 (segment (start 226.91 68.91) (end 226.91 72.9) (width 0.4) (layer "B.Cu") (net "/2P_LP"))
 (segment (start 226.9 46.1) (end 226.91 46.11) (width 0.2) (layer "B.Cu") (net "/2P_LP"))
 (segment (start 226.91 50.296) (end 225.206 52) (width 0.4) (layer "B.Cu") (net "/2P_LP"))
 (segment (start 214.84 62.84) (end 217.414 65.414) (width 0.4) (layer "B.Cu") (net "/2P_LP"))
 (segment (start 226.91 46.09) (end 226.9 46.1) (width 0.2) (layer "B.Cu") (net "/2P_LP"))
 (segment (start 225.206 52) (end 219.1735 52) (width 0.4) (layer "B.Cu") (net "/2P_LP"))
 (segment (start 226.91 46) (end 226.91 46.09) (width 0.2) (layer "B.Cu") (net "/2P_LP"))
 (segment (start 230.87 68.744) (end 230.87 72.9) (width 0.4) (layer "B.Cu") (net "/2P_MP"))
 (segment (start 230.842 46.028) (end 230.842 49.92) (width 0.4) (layer "B.Cu") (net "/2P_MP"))
 (segment (start 216.11 61.35) (end 219.158 64.398) (width 0.4) (layer "B.Cu") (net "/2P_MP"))
 (segment (start 230.842 49.92) (end 227.794 52.968) (width 0.4) (layer "B.Cu") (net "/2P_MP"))
 (segment (start 219.158 64.398) (end 226.524 64.398) (width 0.4) (layer "B.Cu") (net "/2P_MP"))
 (segment (start 230.87 46) (end 230.842 46.028) (width 0.4) (layer "B.Cu") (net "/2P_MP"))
 (segment (start 219.539 52.968) (end 216.11 56.397) (width 0.4) (layer "B.Cu") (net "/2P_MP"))
 (segment (start 216.11 56.397) (end 216.11 61.35) (width 0.4) (layer "B.Cu") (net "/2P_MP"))
 (segment (start 226.524 64.398) (end 230.87 68.744) (width 0.4) (layer "B.Cu") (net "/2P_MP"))
 (segment (start 227.794 52.968) (end 219.539 52.968) (width 0.4) (layer "B.Cu") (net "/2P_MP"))
 (segment (start 242.78 52.46) (end 241.764 53.476) (width 0.4) (layer "B.Cu") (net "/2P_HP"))
 (segment (start 234.83 68.894) (end 234.83 69.91) (width 0.4) (layer "B.Cu") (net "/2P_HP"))
 (segment (start 230.08 53.476) (end 228.048 55.508) (width 0.4) (layer "B.Cu") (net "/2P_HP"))
 (segment (start 241.764 53.476) (end 230.08 53.476) (width 0.4) (layer "B.Cu") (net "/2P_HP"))
 (segment (start 234.83 72.9) (end 234.83 69.91) (width 0.2) (layer "B.Cu") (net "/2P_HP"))
 (segment (start 242.78 46.03) (end 242.78 52.46) (width 0.4) (layer "B.Cu") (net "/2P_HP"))
 (segment (start 218.015 56.27) (end 218.015 60.715) (width 0.4) (layer "B.Cu") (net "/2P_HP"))
 (segment (start 218.777 55.508) (end 218.015 56.27) (width 0.4) (layer "B.Cu") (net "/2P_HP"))
 (segment (start 229.064 63.128) (end 234.83 68.894) (width 0.4) (layer "B.Cu") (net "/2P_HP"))
 (segment (start 220.428 63.128) (end 229.064 63.128) (width 0.4) (layer "B.Cu") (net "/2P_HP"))
 (segment (start 218.015 60.715) (end 220.428 63.128) (width 0.4) (layer "B.Cu") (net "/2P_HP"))
 (segment (start 228.048 55.508) (end 218.777 55.508) (width 0.4) (layer "B.Cu") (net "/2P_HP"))
 (segment (start 242.75 46) (end 242.78 46.03) (width 0.4) (layer "B.Cu") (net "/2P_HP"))
 (segment (start 234.87005 50.998) (end 234.83 50.95795) (width 0.4) (layer "F.Cu") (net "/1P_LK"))
 (segment (start 240.922 54.666) (end 237.254 50.998) (width 0.4) (layer "F.Cu") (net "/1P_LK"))
 (segment (start 234.83 50.95795) (end 234.83 49.51) (width 0.4) (layer "F.Cu") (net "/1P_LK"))
 (segment (start 240.922 60.08) (end 240.922 54.666) (width 0.4) (layer "F.Cu") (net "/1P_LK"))
 (segment (start 237.254 50.998) (end 234.87005 50.998) (width 0.4) (layer "F.Cu") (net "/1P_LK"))
 (segment (start 234.83 49.51) (end 234.83 46) (width 0.2) (layer "F.Cu") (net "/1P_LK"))
 (segment (start 244.558 56.778) (end 238.79 51.01) (width 0.4) (layer "F.Cu") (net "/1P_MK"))
 (segment (start 238.79 51.01) (end 238.79 46) (width 0.4) (layer "F.Cu") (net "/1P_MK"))
 (segment (start 244.812 56.778) (end 244.558 56.778) (width 0.4) (layer "F.Cu") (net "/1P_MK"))
 (segment (start 239.986 56.778) (end 238.422 58.342) (width 0.4) (layer "F.Cu") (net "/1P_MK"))
 (segment (start 238.422 58.342) (end 238.422 60.08) (width 0.4) (layer "F.Cu") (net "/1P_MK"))
 (via (at 239.986 56.778) (size 0.6) (drill 0.3) (layers "F.Cu" "B.Cu") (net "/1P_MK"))
 (via (at 244.812 56.778) (size 0.6) (drill 0.3) (layers "F.Cu" "B.Cu") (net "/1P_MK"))
 (segment (start 244.812 56.778) (end 239.986 56.778) (width 0.4) (layer "B.Cu") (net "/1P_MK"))
 (segment (start 235.922 58.048) (end 235.922 60.08) (width 0.4) (layer "F.Cu") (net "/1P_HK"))
 (segment (start 246.71 53.61) (end 246.71 46) (width 0.4) (layer "F.Cu") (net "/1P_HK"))
 (segment (start 238.462 55.508) (end 235.922 58.048) (width 0.4) (layer "F.Cu") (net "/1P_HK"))
 (segment (start 244.812 55.508) (end 246.71 53.61) (width 0.4) (layer "F.Cu") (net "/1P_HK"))
 (via (at 244.812 55.508) (size 0.6) (drill 0.3) (layers "F.Cu" "B.Cu") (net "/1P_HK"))
 (via (at 238.462 55.508) (size 0.6) (drill 0.3) (layers "F.Cu" "B.Cu") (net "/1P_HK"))
 (segment (start 238.462 55.508) (end 244.812 55.508) (width 0.4) (layer "B.Cu") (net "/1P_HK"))
 (segment (start 233.382 51.76) (end 233.32 51.76) (width 0.4) (layer "F.Cu") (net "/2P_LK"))
 (segment (start 230.842 54.238) (end 230.842 55.508) (width 0.4) (layer "F.Cu") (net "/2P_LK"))
 (segment (start 233.32 51.76) (end 230.842 54.238) (width 0.4) (layer "F.Cu") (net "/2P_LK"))
 (via (at 230.842 55.508) (size 0.6) (drill 0.3) (layers "F.Cu" "B.Cu") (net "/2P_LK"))
 (via (at 233.382 51.76) (size 0.6) (drill 0.3) (layers "F.Cu" "B.Cu") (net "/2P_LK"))
 (segment (start 233.382 51.76) (end 234.336 51.76) (width 0.4) (layer "B.Cu") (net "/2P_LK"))
 (segment (start 230.842 55.508) (end 232.874 55.508) (width 0.4) (layer "B.Cu") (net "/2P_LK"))
 (segment (start 234.83 46) (end 234.83 48.218) (width 0.2) (layer "B.Cu") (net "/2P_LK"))
 (segment (start 232.874 58.048) (end 230.922 60) (width 0.4) (layer "B.Cu") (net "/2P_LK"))
 (segment (start 232.874 55.508) (end 232.874 58.048) (width 0.4) (layer "B.Cu") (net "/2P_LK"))
 (segment (start 230.922 60) (end 230.922 60.08) (width 0.4) (layer "B.Cu") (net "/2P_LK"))
 (segment (start 234.83 51.266) (end 234.83 48.218) (width 0.4) (layer "B.Cu") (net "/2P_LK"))
 (segment (start 234.336 51.76) (end 234.83 51.266) (width 0.4) (layer "B.Cu") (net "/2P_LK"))
 (segment (start 236.43 51.698) (end 231.604 56.524) (width 0.4) (layer "F.Cu") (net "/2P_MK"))
 (via (at 231.604 56.524) (size 0.6) (drill 0.3) (layers "F.Cu" "B.Cu") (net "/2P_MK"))
 (via (at 236.43 51.698) (size 0.6) (drill 0.3) (layers "F.Cu" "B.Cu") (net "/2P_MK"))
 (segment (start 236.43 51.698) (end 238.208 51.698) (width 0.4) (layer "B.Cu") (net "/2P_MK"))
 (segment (start 238.79 51.116) (end 238.79 48.322) (width 0.4) (layer "B.Cu") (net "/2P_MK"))
 (segment (start 228.422 59.706) (end 228.422 60.08) (width 0.4) (layer "B.Cu") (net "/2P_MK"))
 (segment (start 231.604 56.524) (end 228.422 59.706) (width 0.4) (layer "B.Cu") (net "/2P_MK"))
 (segment (start 238.79 46) (end 238.79 48.322) (width 0.2) (layer "B.Cu") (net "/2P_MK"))
 (segment (start 238.208 51.698) (end 238.79 51.116) (width 0.4) (layer "B.Cu") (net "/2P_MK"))
 (segment (start 246.71 46) (end 246.71 48.825) (width 0.2) (layer "B.Cu") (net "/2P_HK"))
 (segment (start 243.542 54.492) (end 230.588 54.492) (width 0.4) (layer "B.Cu") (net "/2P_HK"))
 (segment (start 225.922 59.158) (end 225.922 60.08) (width 0.4) (layer "B.Cu") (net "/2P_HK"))
 (segment (start 246.71 51.324) (end 243.542 54.492) (width 0.4) (layer "B.Cu") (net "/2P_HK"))
 (segment (start 230.588 54.492) (end 225.922 59.158) (width 0.4) (layer "B.Cu") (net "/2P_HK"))
 (segment (start 246.71 48.825) (end 246.71 51.324) (width 0.4) (layer "B.Cu") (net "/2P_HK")))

